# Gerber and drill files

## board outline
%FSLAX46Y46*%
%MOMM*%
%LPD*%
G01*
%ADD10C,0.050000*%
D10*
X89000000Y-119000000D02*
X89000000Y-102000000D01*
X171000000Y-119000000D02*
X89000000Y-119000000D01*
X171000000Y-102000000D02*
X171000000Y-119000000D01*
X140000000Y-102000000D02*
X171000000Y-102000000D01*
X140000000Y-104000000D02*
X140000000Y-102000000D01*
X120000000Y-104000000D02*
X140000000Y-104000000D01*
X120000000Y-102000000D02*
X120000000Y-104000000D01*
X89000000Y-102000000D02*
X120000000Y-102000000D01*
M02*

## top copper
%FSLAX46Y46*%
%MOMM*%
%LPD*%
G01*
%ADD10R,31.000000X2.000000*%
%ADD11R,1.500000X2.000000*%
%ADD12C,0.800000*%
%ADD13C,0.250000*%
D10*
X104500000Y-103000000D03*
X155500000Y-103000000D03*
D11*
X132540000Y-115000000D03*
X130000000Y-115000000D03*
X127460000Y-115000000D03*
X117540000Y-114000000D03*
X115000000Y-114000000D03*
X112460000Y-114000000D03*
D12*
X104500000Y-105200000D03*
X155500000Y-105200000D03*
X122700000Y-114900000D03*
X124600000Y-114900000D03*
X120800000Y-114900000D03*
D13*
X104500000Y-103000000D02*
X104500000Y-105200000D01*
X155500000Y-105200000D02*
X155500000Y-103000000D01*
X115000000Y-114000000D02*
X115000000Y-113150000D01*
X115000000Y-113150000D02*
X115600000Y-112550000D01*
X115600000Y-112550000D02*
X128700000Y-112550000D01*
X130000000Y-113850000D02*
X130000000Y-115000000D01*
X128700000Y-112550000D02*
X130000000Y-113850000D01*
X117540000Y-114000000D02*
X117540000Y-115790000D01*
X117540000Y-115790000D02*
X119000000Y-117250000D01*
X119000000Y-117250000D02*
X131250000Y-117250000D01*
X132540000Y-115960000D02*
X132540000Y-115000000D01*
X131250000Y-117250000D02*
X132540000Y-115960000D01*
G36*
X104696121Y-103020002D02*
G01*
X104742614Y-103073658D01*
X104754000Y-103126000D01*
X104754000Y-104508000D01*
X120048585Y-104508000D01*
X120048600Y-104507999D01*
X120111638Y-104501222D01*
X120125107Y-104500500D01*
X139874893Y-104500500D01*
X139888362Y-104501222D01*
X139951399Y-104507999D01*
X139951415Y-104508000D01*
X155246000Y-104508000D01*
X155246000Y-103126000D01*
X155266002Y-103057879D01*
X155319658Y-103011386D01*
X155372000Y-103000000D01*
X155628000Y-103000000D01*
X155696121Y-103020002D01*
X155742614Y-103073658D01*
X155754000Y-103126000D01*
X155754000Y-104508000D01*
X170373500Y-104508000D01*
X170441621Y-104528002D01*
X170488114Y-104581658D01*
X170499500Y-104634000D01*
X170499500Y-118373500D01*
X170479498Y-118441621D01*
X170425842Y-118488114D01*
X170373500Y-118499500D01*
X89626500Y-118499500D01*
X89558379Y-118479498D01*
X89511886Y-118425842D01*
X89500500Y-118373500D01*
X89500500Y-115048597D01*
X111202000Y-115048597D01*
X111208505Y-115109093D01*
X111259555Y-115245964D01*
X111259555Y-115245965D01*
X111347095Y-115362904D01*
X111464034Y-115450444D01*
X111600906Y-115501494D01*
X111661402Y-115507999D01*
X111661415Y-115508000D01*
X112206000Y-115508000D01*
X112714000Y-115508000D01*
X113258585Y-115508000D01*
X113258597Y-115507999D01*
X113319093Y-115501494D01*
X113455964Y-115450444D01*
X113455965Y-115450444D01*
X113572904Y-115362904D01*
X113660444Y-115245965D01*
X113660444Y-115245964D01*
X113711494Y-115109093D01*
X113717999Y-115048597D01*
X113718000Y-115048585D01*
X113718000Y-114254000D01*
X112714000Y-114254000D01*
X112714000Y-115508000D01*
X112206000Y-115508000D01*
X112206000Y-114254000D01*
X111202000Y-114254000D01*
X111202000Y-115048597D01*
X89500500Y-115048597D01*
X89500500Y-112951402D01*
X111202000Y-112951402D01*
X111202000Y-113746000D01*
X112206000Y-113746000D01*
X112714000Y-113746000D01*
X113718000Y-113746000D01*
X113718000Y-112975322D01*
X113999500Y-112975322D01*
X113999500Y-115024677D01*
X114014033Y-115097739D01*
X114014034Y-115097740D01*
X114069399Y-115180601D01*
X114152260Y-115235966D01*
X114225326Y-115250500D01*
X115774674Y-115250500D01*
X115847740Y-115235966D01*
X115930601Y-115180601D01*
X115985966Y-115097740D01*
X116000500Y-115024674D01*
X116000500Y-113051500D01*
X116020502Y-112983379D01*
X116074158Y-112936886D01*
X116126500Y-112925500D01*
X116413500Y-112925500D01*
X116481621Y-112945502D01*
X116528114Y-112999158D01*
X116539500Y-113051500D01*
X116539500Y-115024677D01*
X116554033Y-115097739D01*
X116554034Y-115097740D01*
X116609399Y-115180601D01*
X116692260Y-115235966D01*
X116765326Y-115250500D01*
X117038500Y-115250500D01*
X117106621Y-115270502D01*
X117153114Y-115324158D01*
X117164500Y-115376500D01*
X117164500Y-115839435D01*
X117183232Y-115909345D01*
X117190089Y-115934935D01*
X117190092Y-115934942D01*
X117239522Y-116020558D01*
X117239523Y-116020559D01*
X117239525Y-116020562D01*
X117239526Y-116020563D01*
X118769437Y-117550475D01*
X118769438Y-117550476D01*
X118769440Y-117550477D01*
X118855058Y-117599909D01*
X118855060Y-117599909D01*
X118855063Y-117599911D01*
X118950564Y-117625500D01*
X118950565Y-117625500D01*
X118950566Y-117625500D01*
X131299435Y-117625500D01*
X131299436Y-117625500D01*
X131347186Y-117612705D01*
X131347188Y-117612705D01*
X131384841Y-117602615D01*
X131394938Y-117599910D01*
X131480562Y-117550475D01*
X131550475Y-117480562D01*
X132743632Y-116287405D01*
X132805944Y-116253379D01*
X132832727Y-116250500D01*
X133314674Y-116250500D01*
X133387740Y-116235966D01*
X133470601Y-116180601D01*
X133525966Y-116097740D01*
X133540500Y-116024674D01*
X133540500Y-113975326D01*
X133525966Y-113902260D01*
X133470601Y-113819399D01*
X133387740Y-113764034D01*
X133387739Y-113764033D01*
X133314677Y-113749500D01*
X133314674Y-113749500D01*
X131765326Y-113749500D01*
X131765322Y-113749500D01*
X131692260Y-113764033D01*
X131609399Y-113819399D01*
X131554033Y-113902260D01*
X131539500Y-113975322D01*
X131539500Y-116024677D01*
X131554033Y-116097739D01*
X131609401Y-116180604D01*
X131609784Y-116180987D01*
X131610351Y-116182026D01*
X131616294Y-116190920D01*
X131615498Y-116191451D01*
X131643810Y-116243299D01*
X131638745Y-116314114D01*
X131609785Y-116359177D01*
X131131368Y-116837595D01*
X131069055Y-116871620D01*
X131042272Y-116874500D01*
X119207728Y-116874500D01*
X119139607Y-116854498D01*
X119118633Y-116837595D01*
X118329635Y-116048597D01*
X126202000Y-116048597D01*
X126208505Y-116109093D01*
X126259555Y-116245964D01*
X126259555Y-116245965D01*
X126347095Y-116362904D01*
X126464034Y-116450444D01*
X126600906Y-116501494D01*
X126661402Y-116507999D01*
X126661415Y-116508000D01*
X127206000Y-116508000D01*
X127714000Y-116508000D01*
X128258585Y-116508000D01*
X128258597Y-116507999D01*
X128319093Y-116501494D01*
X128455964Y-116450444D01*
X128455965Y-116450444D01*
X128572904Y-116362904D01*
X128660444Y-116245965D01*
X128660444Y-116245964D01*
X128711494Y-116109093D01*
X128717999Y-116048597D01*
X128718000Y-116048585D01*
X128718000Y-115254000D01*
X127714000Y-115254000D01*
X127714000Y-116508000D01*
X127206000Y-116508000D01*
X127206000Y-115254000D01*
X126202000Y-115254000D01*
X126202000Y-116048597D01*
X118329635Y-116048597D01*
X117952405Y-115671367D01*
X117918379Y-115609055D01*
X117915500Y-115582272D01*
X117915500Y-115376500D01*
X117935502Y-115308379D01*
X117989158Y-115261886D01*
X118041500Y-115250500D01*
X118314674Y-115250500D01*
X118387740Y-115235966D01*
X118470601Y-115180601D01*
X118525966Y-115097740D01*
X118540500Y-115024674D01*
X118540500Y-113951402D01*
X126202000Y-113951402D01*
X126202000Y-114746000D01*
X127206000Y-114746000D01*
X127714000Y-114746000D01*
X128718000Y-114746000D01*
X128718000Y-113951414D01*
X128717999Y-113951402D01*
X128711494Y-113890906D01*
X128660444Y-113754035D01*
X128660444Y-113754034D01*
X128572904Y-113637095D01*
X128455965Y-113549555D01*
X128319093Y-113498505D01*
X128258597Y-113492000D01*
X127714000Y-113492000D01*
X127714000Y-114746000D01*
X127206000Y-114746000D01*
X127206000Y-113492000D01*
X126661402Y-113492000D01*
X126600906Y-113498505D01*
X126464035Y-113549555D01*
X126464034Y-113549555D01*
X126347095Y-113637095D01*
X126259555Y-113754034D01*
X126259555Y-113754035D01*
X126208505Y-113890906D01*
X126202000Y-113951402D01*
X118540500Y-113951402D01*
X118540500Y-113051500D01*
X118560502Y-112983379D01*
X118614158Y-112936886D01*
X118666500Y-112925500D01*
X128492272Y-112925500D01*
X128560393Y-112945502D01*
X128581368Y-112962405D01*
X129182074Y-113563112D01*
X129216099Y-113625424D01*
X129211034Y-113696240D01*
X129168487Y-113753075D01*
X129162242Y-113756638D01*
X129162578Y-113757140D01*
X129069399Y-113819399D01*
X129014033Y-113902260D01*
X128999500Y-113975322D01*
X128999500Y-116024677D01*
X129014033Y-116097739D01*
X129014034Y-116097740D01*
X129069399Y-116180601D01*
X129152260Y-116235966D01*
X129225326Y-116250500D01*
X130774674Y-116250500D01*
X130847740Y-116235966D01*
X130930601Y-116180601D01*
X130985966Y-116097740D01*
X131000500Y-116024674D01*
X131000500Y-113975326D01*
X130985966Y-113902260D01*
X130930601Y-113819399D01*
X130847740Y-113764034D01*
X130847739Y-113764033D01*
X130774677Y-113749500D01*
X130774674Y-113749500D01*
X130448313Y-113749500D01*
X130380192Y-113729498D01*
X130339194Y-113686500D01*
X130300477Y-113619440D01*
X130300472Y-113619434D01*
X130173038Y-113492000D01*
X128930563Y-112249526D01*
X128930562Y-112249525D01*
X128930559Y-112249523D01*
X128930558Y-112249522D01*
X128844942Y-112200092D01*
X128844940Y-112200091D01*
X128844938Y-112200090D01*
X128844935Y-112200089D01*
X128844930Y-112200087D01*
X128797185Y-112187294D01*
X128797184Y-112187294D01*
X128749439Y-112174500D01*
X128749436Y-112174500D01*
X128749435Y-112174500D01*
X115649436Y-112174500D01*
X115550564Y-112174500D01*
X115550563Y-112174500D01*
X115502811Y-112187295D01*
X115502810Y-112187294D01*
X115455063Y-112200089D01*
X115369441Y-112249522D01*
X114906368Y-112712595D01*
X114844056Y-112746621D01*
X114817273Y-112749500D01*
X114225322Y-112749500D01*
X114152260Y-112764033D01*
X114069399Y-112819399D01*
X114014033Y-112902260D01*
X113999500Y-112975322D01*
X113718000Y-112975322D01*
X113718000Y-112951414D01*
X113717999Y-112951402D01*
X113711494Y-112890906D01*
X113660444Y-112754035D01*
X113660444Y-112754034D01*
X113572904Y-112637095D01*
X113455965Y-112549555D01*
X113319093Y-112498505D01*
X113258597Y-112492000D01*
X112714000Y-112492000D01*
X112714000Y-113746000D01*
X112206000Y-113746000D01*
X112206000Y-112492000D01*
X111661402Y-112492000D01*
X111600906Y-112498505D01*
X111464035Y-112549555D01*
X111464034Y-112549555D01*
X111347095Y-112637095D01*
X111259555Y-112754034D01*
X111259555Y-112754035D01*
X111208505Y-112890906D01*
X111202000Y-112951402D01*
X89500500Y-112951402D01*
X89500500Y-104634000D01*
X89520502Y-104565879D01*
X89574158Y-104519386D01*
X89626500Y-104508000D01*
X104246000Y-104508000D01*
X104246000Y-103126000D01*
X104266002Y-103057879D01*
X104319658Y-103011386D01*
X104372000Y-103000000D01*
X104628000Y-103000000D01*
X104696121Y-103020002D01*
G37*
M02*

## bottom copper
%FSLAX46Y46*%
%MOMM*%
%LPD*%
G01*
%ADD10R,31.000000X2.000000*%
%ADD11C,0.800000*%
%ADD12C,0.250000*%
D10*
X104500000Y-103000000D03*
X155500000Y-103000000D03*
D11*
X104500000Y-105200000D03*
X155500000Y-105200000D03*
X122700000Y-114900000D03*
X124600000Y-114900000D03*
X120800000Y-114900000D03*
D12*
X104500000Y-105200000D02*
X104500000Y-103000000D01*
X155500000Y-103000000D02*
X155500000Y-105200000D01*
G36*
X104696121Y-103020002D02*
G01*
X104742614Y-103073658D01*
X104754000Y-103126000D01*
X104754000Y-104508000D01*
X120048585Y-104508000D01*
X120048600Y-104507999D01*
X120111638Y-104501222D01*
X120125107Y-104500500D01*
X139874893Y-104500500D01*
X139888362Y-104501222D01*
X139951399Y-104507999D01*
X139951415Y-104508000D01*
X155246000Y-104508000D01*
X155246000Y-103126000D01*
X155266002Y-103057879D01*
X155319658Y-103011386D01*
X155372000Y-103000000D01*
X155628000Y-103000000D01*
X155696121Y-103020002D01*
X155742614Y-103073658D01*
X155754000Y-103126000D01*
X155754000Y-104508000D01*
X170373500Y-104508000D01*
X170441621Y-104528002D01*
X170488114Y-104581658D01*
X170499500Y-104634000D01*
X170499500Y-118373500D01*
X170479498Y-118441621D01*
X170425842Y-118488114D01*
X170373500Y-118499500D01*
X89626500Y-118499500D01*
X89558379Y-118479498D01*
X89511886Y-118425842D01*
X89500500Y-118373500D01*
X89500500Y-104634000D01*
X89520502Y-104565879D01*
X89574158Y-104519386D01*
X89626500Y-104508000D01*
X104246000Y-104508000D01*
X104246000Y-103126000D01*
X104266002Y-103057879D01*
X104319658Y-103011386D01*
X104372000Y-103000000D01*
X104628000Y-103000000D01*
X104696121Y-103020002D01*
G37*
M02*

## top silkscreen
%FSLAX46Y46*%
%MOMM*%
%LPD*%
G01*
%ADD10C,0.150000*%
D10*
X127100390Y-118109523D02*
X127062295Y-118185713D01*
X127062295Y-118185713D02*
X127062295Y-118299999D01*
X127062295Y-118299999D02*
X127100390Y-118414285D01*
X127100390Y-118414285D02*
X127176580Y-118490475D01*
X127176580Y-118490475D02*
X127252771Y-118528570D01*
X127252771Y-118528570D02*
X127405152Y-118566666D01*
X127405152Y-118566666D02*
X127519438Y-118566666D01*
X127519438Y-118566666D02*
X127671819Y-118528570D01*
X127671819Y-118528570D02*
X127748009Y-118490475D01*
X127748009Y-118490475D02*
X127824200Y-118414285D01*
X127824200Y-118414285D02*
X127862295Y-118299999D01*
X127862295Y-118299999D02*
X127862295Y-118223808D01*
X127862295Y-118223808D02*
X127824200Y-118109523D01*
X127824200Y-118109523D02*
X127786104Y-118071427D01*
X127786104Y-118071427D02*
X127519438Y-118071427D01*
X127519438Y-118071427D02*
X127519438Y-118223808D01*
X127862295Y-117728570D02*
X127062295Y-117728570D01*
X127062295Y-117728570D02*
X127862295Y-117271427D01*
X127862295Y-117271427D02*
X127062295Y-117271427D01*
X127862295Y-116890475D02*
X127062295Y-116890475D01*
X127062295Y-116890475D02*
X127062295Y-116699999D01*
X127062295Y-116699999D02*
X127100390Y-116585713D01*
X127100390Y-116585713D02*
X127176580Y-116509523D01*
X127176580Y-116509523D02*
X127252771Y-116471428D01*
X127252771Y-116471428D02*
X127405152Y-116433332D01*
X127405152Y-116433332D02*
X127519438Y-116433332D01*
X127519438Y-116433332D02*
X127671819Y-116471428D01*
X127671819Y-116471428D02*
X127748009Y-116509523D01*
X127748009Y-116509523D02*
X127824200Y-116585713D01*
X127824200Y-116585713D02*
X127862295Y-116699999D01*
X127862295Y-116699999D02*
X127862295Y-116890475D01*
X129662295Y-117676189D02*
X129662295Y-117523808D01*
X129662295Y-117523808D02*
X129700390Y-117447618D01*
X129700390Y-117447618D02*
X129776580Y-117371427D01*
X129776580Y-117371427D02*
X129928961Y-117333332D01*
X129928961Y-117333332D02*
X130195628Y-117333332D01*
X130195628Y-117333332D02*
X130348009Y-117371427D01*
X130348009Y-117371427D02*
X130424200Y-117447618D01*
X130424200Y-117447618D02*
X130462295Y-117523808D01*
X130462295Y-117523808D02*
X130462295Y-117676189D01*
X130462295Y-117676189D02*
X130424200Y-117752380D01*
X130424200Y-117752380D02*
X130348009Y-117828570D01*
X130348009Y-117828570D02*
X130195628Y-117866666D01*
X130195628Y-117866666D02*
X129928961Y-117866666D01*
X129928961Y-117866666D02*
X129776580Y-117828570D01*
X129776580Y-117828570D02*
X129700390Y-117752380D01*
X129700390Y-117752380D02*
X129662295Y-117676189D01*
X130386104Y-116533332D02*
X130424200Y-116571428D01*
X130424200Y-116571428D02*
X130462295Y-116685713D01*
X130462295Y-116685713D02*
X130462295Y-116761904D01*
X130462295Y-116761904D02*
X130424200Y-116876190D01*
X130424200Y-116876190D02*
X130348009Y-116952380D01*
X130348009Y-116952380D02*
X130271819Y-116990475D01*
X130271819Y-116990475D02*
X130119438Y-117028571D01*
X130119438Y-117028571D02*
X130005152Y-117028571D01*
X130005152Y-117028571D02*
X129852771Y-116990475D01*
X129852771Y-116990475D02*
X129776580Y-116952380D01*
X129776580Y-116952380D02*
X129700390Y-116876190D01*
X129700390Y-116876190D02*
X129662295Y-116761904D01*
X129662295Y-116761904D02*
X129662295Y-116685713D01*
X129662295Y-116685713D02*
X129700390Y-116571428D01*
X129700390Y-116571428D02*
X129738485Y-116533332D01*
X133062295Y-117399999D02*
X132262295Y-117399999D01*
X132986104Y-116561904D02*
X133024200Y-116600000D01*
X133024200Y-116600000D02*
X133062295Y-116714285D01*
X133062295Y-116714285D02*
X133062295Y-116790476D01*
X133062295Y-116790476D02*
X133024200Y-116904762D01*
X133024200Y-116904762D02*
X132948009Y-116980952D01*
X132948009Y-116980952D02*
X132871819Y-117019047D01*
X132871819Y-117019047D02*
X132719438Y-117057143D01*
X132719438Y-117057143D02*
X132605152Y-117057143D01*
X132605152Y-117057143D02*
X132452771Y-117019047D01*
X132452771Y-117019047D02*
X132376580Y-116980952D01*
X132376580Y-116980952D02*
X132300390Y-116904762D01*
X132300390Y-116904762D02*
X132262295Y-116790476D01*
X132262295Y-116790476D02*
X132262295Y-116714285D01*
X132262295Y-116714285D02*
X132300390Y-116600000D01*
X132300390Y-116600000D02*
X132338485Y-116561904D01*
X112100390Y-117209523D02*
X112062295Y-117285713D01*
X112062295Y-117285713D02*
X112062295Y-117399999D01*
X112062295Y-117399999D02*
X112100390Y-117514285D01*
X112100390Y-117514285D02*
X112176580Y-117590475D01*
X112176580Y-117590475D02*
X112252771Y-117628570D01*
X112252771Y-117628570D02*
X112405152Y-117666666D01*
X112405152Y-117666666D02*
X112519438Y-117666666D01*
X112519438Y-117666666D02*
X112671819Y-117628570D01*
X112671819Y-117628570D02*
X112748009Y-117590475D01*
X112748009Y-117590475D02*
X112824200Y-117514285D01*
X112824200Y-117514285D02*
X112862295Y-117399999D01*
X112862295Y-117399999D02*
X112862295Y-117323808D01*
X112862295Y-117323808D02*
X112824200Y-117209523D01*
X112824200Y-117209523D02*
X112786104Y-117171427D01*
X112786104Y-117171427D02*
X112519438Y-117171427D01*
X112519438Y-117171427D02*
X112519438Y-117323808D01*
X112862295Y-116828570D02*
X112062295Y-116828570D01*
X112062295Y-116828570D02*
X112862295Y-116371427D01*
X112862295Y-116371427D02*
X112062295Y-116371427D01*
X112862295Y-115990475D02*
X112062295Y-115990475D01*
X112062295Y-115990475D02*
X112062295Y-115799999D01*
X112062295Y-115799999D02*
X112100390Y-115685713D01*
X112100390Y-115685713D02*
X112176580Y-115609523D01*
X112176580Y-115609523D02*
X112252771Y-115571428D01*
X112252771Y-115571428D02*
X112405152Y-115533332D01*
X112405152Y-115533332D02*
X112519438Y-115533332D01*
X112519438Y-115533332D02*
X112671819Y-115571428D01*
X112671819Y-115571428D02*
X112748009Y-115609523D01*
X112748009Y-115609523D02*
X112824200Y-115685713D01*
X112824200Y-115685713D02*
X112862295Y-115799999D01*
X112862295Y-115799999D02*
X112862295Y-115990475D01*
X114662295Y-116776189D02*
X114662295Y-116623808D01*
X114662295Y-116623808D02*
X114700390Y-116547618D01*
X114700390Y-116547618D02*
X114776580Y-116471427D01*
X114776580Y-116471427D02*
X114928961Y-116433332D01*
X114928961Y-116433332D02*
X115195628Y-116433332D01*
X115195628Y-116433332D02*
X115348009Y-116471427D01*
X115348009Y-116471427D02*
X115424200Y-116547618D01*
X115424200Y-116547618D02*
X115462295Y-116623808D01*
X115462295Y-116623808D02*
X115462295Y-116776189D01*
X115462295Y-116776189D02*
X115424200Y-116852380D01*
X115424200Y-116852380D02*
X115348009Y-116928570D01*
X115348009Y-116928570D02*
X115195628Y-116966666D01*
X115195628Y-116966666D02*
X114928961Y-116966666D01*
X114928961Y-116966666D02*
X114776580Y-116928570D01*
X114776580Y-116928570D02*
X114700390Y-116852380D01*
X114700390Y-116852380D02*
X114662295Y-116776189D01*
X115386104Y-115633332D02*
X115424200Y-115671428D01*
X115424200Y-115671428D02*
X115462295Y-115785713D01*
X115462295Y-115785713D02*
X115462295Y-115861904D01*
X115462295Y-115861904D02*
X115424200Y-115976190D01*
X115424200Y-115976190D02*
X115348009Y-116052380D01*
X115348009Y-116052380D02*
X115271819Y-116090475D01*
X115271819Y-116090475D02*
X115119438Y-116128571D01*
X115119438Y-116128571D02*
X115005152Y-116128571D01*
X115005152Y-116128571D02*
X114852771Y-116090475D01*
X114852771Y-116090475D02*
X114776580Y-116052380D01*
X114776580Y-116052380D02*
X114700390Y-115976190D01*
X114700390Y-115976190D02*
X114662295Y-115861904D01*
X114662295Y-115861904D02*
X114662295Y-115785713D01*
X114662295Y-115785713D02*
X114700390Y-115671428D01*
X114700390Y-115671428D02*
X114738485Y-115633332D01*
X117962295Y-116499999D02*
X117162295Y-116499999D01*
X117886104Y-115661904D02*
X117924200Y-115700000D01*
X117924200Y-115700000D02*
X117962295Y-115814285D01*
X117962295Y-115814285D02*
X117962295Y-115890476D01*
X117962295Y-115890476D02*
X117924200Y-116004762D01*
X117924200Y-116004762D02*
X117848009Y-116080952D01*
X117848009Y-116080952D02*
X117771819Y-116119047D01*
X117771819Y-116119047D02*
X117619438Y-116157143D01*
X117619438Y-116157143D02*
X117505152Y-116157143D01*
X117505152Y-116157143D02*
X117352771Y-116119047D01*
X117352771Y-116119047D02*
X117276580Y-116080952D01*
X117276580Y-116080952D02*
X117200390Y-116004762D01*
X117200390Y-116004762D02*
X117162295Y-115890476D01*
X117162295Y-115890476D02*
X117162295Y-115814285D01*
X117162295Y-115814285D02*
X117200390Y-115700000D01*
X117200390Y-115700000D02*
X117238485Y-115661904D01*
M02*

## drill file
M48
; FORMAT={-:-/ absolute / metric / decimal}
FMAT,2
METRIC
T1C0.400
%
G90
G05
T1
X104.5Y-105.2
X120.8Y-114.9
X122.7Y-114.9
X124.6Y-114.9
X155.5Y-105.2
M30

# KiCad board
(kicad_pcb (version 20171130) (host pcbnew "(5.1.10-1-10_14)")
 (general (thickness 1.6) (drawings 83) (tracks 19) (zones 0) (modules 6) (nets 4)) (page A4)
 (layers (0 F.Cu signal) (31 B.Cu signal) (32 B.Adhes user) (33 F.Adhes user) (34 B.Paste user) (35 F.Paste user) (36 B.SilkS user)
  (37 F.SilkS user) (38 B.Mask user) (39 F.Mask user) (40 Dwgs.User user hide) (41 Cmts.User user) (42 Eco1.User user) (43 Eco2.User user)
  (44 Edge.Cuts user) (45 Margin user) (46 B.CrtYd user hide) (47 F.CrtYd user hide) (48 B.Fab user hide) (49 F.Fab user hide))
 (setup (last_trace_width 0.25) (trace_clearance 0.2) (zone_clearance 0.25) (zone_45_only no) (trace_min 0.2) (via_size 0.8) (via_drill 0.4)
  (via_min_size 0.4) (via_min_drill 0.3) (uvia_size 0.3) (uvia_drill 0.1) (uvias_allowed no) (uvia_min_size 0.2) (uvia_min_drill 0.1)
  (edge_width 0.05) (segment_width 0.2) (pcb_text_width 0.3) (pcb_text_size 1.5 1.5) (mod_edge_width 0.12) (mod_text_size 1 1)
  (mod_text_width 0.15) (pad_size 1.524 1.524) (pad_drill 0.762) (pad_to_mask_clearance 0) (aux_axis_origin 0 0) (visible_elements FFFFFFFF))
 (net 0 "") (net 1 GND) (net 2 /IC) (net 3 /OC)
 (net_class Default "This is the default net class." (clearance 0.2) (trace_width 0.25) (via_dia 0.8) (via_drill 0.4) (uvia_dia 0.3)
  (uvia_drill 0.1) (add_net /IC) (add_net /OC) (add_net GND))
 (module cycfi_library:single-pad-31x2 (layer F.Cu) (at 104.5 103)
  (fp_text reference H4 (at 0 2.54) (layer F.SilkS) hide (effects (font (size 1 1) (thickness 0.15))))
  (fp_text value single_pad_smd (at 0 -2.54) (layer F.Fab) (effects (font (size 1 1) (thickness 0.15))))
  (pad 1 smd rect (at 0 0) (size 31 2) (layers F.Cu F.Paste F.Mask) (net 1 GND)))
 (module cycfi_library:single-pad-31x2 (layer B.Cu) (at 104.5 103)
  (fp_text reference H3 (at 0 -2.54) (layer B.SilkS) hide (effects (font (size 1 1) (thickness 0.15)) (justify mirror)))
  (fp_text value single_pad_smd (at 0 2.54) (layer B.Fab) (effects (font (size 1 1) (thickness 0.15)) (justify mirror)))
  (pad 1 smd rect (at 0 0) (size 31 2) (layers B.Cu B.Paste B.Mask) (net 1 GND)))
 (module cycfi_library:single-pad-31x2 (layer F.Cu) (at 155.5 103)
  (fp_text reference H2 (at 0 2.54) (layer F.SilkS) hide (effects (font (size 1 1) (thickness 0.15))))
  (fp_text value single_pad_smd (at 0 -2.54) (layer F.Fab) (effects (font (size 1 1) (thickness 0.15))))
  (pad 1 smd rect (at 0 0) (size 31 2) (layers F.Cu F.Paste F.Mask) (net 1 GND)))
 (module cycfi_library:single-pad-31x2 (layer B.Cu) (at 155.5 103)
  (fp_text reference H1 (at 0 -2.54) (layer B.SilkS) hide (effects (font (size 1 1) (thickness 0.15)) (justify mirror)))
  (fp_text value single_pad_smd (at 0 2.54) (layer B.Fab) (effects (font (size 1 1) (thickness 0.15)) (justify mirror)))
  (pad 1 smd rect (at 0 0) (size 31 2) (layers B.Cu B.Paste B.Mask) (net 1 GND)))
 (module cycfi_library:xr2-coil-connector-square (layer F.Cu) (at 130 115)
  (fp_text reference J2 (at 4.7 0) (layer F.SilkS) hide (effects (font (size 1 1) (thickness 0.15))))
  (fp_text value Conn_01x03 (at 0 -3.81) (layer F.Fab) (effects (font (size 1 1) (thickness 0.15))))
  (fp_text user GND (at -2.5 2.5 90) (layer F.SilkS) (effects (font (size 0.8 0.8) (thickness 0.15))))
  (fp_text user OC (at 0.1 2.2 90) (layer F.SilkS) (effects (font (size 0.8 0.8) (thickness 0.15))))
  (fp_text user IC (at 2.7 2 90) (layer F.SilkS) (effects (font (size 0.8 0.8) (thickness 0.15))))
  (pad 3 smd rect (at 2.54 0) (size 1.5 2) (layers F.Cu F.Paste F.Mask) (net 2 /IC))
  (pad 2 smd rect (at 0 0) (size 1.5 2) (layers F.Cu F.Paste F.Mask) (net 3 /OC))
  (pad 1 smd rect (at -2.54 0) (size 1.5 2) (layers F.Cu F.Paste F.Mask) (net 1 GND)))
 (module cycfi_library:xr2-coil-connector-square (layer F.Cu) (at 115 114)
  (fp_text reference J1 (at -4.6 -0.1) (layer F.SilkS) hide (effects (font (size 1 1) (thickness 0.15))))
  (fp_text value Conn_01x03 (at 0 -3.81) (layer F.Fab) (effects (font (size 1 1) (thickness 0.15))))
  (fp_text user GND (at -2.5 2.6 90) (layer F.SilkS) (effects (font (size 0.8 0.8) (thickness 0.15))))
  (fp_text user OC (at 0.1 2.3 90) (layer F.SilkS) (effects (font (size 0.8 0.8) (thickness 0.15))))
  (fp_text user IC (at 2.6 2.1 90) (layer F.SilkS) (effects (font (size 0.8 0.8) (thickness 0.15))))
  (pad 3 smd rect (at 2.54 0) (size 1.5 2) (layers F.Cu F.Paste F.Mask) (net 2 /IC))
  (pad 2 smd rect (at 0 0) (size 1.5 2) (layers F.Cu F.Paste F.Mask) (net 3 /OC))
  (pad 1 smd rect (at -2.54 0) (size 1.5 2) (layers F.Cu F.Paste F.Mask) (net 1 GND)))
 (gr_line (start 89 119) (end 89 102) (layer Edge.Cuts) (width 0.05))
 (gr_line (start 171 119) (end 89 119) (layer Edge.Cuts) (width 0.05))
 (gr_line (start 171 102) (end 171 119) (layer Edge.Cuts) (width 0.05))
 (gr_line (start 140 102) (end 171 102) (layer Edge.Cuts) (width 0.05))
 (gr_line (start 140 104) (end 140 102) (layer Edge.Cuts) (width 0.05))
 (gr_line (start 120 104) (end 140 104) (layer Edge.Cuts) (width 0.05))
 (gr_line (start 120 102) (end 120 104) (layer Edge.Cuts) (width 0.05))
 (gr_line (start 89 102) (end 120 102) (layer Edge.Cuts) (width 0.05))
 (via (at 104.5 105.2) (size 0.8) (drill 0.4) (layers F.Cu B.Cu) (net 1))
 (segment (start 104.5 103) (end 104.5 105.2) (width 0.25) (layer F.Cu) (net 1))
 (segment (start 104.5 105.2) (end 104.5 103) (width 0.25) (layer B.Cu) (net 1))
 (via (at 155.5 105.2) (size 0.8) (drill 0.4) (layers F.Cu B.Cu) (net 1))
 (segment (start 155.5 103) (end 155.5 105.2) (width 0.25) (layer B.Cu) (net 1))
 (segment (start 155.5 105.2) (end 155.5 103) (width 0.25) (layer F.Cu) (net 1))
 (via (at 122.7 114.9) (size 0.8) (drill 0.4) (layers F.Cu B.Cu) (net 1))
 (via (at 124.6 114.9) (size 0.8) (drill 0.4) (layers F.Cu B.Cu) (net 1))
 (via (at 120.8 114.9) (size 0.8) (drill 0.4) (layers F.Cu B.Cu) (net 1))
 (segment (start 115 114) (end 115 113.15) (width 0.25) (layer F.Cu) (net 3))
 (segment (start 115 113.15) (end 115.6 112.55) (width 0.25) (layer F.Cu) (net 3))
 (segment (start 115.6 112.55) (end 128.7 112.55) (width 0.25) (layer F.Cu) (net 3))
 (segment (start 130 113.85) (end 130 115) (width 0.25) (layer F.Cu) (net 3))
 (segment (start 128.7 112.55) (end 130 113.85) (width 0.25) (layer F.Cu) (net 3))
 (segment (start 117.54 114) (end 117.54 115.79) (width 0.25) (layer F.Cu) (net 2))
 (segment (start 117.54 115.79) (end 119 117.25) (width 0.25) (layer F.Cu) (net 2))
 (segment (start 119 117.25) (end 131.25 117.25) (width 0.25) (layer F.Cu) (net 2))
 (segment (start 132.54 115.96) (end 132.54 115) (width 0.25) (layer F.Cu) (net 2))
 (segment (start 131.25 117.25) (end 132.54 115.96) (width 0.25) (layer F.Cu) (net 2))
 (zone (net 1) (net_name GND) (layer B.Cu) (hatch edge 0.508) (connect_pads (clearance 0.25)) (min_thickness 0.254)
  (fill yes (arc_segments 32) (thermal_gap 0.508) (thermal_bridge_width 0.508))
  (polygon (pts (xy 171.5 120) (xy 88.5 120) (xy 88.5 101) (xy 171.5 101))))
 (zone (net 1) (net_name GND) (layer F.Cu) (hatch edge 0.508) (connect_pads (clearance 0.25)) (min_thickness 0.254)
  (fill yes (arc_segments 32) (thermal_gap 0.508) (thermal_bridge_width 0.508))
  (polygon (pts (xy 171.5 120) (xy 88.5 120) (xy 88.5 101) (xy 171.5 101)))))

